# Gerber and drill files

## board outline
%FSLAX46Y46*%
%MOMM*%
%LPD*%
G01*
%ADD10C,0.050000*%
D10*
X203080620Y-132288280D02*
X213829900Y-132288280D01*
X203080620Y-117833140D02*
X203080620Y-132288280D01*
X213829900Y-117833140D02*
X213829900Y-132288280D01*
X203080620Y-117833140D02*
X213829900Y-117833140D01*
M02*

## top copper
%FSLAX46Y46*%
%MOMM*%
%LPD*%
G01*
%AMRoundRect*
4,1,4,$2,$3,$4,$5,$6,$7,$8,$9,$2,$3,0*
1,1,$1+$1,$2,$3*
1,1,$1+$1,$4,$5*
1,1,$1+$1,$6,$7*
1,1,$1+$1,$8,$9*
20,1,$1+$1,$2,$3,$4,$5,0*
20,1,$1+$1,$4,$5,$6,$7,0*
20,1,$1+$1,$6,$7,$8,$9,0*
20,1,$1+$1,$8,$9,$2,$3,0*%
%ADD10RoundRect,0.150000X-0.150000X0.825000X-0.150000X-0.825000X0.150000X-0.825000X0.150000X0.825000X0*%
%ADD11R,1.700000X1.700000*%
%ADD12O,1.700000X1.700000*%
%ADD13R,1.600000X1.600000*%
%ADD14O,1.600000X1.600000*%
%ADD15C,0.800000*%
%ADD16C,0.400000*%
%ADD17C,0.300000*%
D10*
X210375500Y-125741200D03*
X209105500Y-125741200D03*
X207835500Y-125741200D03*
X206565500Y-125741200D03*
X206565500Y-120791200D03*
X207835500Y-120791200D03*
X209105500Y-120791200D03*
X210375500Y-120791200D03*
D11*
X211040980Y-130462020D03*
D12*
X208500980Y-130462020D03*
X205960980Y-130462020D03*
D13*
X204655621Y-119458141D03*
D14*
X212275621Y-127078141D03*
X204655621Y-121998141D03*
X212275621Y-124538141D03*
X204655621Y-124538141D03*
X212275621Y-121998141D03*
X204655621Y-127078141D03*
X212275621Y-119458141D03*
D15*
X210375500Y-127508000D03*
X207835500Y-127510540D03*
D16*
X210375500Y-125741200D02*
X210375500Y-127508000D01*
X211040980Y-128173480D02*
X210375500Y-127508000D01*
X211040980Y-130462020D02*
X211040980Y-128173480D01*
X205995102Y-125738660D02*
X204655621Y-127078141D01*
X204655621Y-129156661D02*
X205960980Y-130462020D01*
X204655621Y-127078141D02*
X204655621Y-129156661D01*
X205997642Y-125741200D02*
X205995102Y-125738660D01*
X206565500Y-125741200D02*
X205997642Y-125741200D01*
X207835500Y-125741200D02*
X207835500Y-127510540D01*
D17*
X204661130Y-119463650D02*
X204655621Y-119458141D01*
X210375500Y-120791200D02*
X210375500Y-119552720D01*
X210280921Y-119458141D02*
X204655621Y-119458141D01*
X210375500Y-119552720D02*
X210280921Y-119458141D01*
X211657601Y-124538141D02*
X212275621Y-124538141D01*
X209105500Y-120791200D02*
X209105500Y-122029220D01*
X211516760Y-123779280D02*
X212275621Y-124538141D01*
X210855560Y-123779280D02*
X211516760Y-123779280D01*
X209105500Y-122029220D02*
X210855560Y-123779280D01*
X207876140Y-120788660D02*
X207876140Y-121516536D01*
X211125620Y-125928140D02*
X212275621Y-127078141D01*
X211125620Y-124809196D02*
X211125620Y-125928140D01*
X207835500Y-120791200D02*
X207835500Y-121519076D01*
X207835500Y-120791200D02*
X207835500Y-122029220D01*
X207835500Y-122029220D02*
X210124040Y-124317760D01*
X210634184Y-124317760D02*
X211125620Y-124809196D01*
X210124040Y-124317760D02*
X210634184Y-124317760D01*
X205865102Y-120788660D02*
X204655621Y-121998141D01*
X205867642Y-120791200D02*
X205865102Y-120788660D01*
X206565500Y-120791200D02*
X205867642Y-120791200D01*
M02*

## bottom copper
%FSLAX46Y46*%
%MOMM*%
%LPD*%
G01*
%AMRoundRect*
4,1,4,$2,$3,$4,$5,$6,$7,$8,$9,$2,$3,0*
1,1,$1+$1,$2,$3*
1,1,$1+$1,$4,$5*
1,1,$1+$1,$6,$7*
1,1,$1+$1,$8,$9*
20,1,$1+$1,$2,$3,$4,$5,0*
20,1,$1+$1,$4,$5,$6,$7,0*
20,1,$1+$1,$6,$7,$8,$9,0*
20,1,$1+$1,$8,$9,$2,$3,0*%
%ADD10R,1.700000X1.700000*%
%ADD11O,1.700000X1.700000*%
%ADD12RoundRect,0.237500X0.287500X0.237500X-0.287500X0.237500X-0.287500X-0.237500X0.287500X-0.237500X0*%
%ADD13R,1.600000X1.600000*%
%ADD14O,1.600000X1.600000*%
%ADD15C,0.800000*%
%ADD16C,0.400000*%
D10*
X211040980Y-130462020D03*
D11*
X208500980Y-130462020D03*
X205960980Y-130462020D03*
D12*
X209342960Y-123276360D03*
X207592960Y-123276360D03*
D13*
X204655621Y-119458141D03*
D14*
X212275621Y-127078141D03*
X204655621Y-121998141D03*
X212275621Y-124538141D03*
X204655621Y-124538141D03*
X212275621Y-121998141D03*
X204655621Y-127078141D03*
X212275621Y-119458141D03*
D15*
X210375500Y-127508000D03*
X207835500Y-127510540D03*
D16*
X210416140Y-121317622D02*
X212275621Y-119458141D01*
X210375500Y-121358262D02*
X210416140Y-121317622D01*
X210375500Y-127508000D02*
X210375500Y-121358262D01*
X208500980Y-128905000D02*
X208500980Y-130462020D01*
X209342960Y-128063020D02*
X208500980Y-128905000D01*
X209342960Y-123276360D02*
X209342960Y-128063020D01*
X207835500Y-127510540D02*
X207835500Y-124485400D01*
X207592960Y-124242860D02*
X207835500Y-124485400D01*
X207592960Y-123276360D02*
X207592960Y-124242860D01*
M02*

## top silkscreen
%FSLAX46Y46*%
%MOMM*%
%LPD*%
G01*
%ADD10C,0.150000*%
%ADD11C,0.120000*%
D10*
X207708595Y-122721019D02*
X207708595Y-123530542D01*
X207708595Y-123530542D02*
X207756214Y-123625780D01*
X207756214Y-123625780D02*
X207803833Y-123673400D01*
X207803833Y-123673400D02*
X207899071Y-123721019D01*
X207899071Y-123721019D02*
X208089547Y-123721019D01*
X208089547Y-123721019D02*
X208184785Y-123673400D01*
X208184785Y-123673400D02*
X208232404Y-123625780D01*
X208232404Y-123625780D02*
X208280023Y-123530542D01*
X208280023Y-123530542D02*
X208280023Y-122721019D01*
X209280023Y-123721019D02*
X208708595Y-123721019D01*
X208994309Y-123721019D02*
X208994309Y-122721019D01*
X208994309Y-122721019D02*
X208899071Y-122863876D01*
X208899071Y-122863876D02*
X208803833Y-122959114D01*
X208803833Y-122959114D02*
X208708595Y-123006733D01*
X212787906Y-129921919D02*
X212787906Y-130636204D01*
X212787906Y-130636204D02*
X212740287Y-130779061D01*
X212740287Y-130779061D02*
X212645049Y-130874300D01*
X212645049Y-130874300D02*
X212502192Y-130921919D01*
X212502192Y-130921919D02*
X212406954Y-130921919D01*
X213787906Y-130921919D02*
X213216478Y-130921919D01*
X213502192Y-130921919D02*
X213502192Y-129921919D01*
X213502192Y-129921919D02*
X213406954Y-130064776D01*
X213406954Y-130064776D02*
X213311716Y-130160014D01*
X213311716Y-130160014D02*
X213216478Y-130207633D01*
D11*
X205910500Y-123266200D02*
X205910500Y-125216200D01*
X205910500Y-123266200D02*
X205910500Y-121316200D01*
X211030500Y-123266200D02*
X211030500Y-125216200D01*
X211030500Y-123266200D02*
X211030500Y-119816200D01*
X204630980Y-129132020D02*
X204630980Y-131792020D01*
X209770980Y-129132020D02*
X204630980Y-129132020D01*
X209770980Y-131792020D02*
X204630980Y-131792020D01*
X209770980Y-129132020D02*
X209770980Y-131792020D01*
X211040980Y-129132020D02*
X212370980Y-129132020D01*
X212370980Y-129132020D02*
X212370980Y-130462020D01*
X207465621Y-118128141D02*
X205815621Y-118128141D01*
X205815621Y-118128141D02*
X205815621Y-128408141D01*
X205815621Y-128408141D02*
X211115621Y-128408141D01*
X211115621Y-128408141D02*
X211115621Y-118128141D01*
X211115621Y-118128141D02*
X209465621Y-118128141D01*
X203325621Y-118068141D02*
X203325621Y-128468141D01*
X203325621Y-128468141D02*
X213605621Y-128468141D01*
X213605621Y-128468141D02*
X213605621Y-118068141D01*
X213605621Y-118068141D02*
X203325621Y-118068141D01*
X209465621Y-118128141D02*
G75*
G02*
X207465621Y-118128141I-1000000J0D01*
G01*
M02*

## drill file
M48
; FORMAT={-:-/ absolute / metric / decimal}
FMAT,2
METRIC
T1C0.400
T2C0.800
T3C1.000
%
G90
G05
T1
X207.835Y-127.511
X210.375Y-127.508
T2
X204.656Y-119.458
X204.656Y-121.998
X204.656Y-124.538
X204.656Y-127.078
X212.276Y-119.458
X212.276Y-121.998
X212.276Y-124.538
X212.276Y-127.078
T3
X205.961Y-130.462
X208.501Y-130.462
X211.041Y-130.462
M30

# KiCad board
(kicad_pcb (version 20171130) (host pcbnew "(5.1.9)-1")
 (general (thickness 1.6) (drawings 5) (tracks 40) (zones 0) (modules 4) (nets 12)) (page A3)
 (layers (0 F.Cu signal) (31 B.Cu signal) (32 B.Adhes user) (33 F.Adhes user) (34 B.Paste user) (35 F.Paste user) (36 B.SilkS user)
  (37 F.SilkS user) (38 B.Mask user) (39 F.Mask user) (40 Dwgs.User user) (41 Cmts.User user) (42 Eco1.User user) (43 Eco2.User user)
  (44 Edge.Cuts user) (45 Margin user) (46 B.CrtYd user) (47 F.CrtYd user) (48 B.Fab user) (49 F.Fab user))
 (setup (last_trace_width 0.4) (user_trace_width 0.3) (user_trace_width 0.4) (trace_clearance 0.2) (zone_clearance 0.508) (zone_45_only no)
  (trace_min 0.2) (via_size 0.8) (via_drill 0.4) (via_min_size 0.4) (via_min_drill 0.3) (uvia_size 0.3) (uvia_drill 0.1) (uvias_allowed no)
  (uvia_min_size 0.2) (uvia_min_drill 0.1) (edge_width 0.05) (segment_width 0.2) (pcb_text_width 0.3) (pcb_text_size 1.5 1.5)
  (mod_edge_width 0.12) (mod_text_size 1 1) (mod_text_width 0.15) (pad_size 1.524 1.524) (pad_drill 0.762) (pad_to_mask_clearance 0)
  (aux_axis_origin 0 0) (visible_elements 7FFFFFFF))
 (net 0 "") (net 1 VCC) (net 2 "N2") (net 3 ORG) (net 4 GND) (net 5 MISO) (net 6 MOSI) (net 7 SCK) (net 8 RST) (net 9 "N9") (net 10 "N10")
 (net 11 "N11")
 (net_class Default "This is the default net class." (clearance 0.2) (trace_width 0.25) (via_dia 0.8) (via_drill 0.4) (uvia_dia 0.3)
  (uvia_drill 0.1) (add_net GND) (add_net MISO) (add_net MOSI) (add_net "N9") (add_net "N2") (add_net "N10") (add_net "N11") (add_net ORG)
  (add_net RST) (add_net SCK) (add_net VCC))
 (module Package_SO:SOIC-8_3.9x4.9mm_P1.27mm (layer F.Cu) (at 208.4705 123.2662 270)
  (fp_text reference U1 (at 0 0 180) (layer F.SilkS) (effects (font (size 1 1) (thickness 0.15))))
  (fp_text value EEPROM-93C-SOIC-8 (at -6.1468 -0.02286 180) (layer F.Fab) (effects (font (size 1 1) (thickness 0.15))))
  (fp_line (start 0 2.56) (end 1.95 2.56) (layer F.SilkS) (width 0.12))
  (fp_line (start 0 2.56) (end -1.95 2.56) (layer F.SilkS) (width 0.12))
  (fp_line (start 0 -2.56) (end 1.95 -2.56) (layer F.SilkS) (width 0.12))
  (fp_line (start 0 -2.56) (end -3.45 -2.56) (layer F.SilkS) (width 0.12))
  (pad 8 smd roundrect (at 2.475 -1.905 270) (size 1.95 0.6) (layers F.Cu F.Paste F.Mask) (roundrect_rratio 0.25) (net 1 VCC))
  (pad 7 smd roundrect (at 2.475 -0.635 270) (size 1.95 0.6) (layers F.Cu F.Paste F.Mask) (roundrect_rratio 0.25) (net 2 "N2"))
  (pad 6 smd roundrect (at 2.475 0.635 270) (size 1.95 0.6) (layers F.Cu F.Paste F.Mask) (roundrect_rratio 0.25) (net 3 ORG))
  (pad 5 smd roundrect (at 2.475 1.905 270) (size 1.95 0.6) (layers F.Cu F.Paste F.Mask) (roundrect_rratio 0.25) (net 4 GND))
  (pad 4 smd roundrect (at -2.475 1.905 270) (size 1.95 0.6) (layers F.Cu F.Paste F.Mask) (roundrect_rratio 0.25) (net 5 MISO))
  (pad 3 smd roundrect (at -2.475 0.635 270) (size 1.95 0.6) (layers F.Cu F.Paste F.Mask) (roundrect_rratio 0.25) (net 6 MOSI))
  (pad 2 smd roundrect (at -2.475 -0.635 270) (size 1.95 0.6) (layers F.Cu F.Paste F.Mask) (roundrect_rratio 0.25) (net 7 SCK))
  (pad 1 smd roundrect (at -2.475 -1.905 270) (size 1.95 0.6) (layers F.Cu F.Paste F.Mask) (roundrect_rratio 0.25) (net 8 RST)))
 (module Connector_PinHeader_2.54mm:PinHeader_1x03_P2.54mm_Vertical (layer F.Cu) (at 211.04098 130.46202 270)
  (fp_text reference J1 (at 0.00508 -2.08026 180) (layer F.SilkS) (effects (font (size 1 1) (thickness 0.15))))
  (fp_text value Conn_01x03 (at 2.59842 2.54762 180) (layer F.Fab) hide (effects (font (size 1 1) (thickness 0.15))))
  (fp_line (start -1.33 6.41) (end 1.33 6.41) (layer F.SilkS) (width 0.12))
  (fp_line (start -1.33 1.27) (end -1.33 6.41) (layer F.SilkS) (width 0.12))
  (fp_line (start 1.33 1.27) (end 1.33 6.41) (layer F.SilkS) (width 0.12))
  (fp_line (start -1.33 1.27) (end 1.33 1.27) (layer F.SilkS) (width 0.12))
  (fp_line (start -1.33 0) (end -1.33 -1.33) (layer F.SilkS) (width 0.12))
  (fp_line (start -1.33 -1.33) (end 0 -1.33) (layer F.SilkS) (width 0.12))
  (pad 1 thru_hole rect (at 0 0 270) (size 1.7 1.7) (drill 1) (layers *.Cu *.Mask) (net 1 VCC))
  (pad 2 thru_hole oval (at 0 2.54 270) (size 1.7 1.7) (drill 1) (layers *.Cu *.Mask) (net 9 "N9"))
  (pad 3 thru_hole oval (at 0 5.08 270) (size 1.7 1.7) (drill 1) (layers *.Cu *.Mask) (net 4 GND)))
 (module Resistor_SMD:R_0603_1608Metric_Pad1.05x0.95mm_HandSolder (layer B.Cu) (at 208.46796 123.27636 180)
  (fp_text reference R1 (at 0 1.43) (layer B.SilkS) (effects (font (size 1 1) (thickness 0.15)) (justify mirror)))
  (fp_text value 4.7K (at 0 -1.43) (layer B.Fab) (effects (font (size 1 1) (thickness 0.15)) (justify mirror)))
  (pad 1 smd roundrect (at -0.875 0 180) (size 1.05 0.95) (layers B.Cu B.Paste B.Mask) (roundrect_rratio 0.25) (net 9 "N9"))
  (pad 2 smd roundrect (at 0.875 0 180) (size 1.05 0.95) (layers B.Cu B.Paste B.Mask) (roundrect_rratio 0.25) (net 3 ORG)))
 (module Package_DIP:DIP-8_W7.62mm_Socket (layer F.Cu) (at 204.655621 119.458141)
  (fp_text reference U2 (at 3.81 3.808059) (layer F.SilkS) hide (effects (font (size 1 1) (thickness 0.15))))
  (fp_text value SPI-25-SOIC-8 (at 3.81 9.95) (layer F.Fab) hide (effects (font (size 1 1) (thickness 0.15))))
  (fp_line (start 2.81 -1.33) (end 1.16 -1.33) (layer F.SilkS) (width 0.12))
  (fp_line (start 1.16 -1.33) (end 1.16 8.95) (layer F.SilkS) (width 0.12))
  (fp_line (start 1.16 8.95) (end 6.46 8.95) (layer F.SilkS) (width 0.12))
  (fp_line (start 6.46 8.95) (end 6.46 -1.33) (layer F.SilkS) (width 0.12))
  (fp_line (start 6.46 -1.33) (end 4.81 -1.33) (layer F.SilkS) (width 0.12))
  (fp_line (start -1.33 -1.39) (end -1.33 9.01) (layer F.SilkS) (width 0.12))
  (fp_line (start -1.33 9.01) (end 8.95 9.01) (layer F.SilkS) (width 0.12))
  (fp_line (start 8.95 9.01) (end 8.95 -1.39) (layer F.SilkS) (width 0.12))
  (fp_line (start 8.95 -1.39) (end -1.33 -1.39) (layer F.SilkS) (width 0.12))
  (fp_arc (start 3.81 -1.33) (end 2.81 -1.33) (angle -180) (layer F.SilkS) (width 0.12))
  (pad 1 thru_hole rect (at 0 0) (size 1.6 1.6) (drill 0.8) (layers *.Cu *.Mask) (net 8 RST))
  (pad 5 thru_hole oval (at 7.62 7.62) (size 1.6 1.6) (drill 0.8) (layers *.Cu *.Mask) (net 6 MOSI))
  (pad 2 thru_hole oval (at 0 2.54) (size 1.6 1.6) (drill 0.8) (layers *.Cu *.Mask) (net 5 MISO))
  (pad 6 thru_hole oval (at 7.62 5.08) (size 1.6 1.6) (drill 0.8) (layers *.Cu *.Mask) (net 7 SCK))
  (pad 3 thru_hole oval (at 0 5.08) (size 1.6 1.6) (drill 0.8) (layers *.Cu *.Mask) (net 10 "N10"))
  (pad 7 thru_hole oval (at 7.62 2.54) (size 1.6 1.6) (drill 0.8) (layers *.Cu *.Mask) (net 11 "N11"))
  (pad 4 thru_hole oval (at 0 7.62) (size 1.6 1.6) (drill 0.8) (layers *.Cu *.Mask) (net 4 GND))
  (pad 8 thru_hole oval (at 7.62 0) (size 1.6 1.6) (drill 0.8) (layers *.Cu *.Mask) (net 1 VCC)))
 (gr_line (start 203.08062 132.28828) (end 213.8299 132.28828) (layer Edge.Cuts) (width 0.05))
 (gr_line (start 203.08062 117.83314) (end 203.08062 132.28828) (layer Edge.Cuts) (width 0.05))
 (gr_line (start 213.8299 117.83314) (end 213.8299 132.28828) (layer Edge.Cuts) (width 0.05))
 (gr_line (start 203.08062 117.83314) (end 213.8299 117.83314) (layer Edge.Cuts) (width 0.05))
 (segment (start 210.41614 121.317622) (end 212.275621 119.458141) (width 0.4) (layer B.Cu) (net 1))
 (segment (start 210.3755 125.7412) (end 210.3755 127.508) (width 0.4) (layer F.Cu) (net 1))
 (via (at 210.3755 127.508) (size 0.8) (drill 0.4) (layers F.Cu B.Cu) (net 1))
 (segment (start 211.04098 128.17348) (end 210.3755 127.508) (width 0.4) (layer F.Cu) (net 1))
 (segment (start 211.04098 130.46202) (end 211.04098 128.17348) (width 0.4) (layer F.Cu) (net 1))
 (segment (start 210.3755 121.358262) (end 210.41614 121.317622) (width 0.4) (layer B.Cu) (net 1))
 (segment (start 210.3755 127.508) (end 210.3755 121.358262) (width 0.4) (layer B.Cu) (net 1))
 (segment (start 208.50098 128.905) (end 208.50098 130.46202) (width 0.4) (layer B.Cu) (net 9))
 (segment (start 209.34296 128.06302) (end 208.50098 128.905) (width 0.4) (layer B.Cu) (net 9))
 (segment (start 209.34296 123.27636) (end 209.34296 128.06302) (width 0.4) (layer B.Cu) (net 9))
 (segment (start 205.995102 125.73866) (end 204.655621 127.078141) (width 0.4) (layer F.Cu) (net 4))
 (segment (start 204.655621 129.156661) (end 205.96098 130.46202) (width 0.4) (layer F.Cu) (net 4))
 (segment (start 204.655621 127.078141) (end 204.655621 129.156661) (width 0.4) (layer F.Cu) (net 4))
 (segment (start 205.997642 125.7412) (end 205.995102 125.73866) (width 0.4) (layer F.Cu) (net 4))
 (segment (start 206.5655 125.7412) (end 205.997642 125.7412) (width 0.4) (layer F.Cu) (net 4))
 (segment (start 207.8355 125.7412) (end 207.8355 127.51054) (width 0.4) (layer F.Cu) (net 3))
 (via (at 207.8355 127.51054) (size 0.8) (drill 0.4) (layers F.Cu B.Cu) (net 3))
 (segment (start 207.8355 127.51054) (end 207.8355 124.4854) (width 0.4) (layer B.Cu) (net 3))
 (segment (start 207.59296 124.24286) (end 207.8355 124.4854) (width 0.4) (layer B.Cu) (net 3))
 (segment (start 207.59296 123.27636) (end 207.59296 124.24286) (width 0.4) (layer B.Cu) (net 3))
 (segment (start 204.66113 119.46365) (end 204.655621 119.458141) (width 0.3) (layer F.Cu) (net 8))
 (segment (start 210.3755 120.7912) (end 210.3755 119.55272) (width 0.3) (layer F.Cu) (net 8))
 (segment (start 210.280921 119.458141) (end 204.655621 119.458141) (width 0.3) (layer F.Cu) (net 8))
 (segment (start 210.3755 119.55272) (end 210.280921 119.458141) (width 0.3) (layer F.Cu) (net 8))
 (segment (start 211.657601 124.538141) (end 212.275621 124.538141) (width 0.3) (layer F.Cu) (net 7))
 (segment (start 209.1055 120.7912) (end 209.1055 122.02922) (width 0.3) (layer F.Cu) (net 7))
 (segment (start 211.51676 123.77928) (end 212.275621 124.538141) (width 0.3) (layer F.Cu) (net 7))
 (segment (start 210.85556 123.77928) (end 211.51676 123.77928) (width 0.3) (layer F.Cu) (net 7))
 (segment (start 209.1055 122.02922) (end 210.85556 123.77928) (width 0.3) (layer F.Cu) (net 7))
 (segment (start 207.87614 120.78866) (end 207.87614 121.516536) (width 0.3) (layer F.Cu) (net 6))
 (segment (start 211.12562 125.92814) (end 212.275621 127.078141) (width 0.3) (layer F.Cu) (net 6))
 (segment (start 211.12562 124.809196) (end 211.12562 125.92814) (width 0.3) (layer F.Cu) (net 6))
 (segment (start 207.8355 120.7912) (end 207.8355 121.519076) (width 0.3) (layer F.Cu) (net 6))
 (segment (start 207.8355 120.7912) (end 207.8355 122.02922) (width 0.3) (layer F.Cu) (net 6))
 (segment (start 207.8355 122.02922) (end 210.12404 124.31776) (width 0.3) (layer F.Cu) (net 6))
 (segment (start 210.634184 124.31776) (end 211.12562 124.809196) (width 0.3) (layer F.Cu) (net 6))
 (segment (start 210.12404 124.31776) (end 210.634184 124.31776) (width 0.3) (layer F.Cu) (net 6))
 (segment (start 205.865102 120.78866) (end 204.655621 121.998141) (width 0.3) (layer F.Cu) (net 5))
 (segment (start 205.867642 120.7912) (end 205.865102 120.78866) (width 0.3) (layer F.Cu) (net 5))
 (segment (start 206.5655 120.7912) (end 205.867642 120.7912) (width 0.3) (layer F.Cu) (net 5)))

